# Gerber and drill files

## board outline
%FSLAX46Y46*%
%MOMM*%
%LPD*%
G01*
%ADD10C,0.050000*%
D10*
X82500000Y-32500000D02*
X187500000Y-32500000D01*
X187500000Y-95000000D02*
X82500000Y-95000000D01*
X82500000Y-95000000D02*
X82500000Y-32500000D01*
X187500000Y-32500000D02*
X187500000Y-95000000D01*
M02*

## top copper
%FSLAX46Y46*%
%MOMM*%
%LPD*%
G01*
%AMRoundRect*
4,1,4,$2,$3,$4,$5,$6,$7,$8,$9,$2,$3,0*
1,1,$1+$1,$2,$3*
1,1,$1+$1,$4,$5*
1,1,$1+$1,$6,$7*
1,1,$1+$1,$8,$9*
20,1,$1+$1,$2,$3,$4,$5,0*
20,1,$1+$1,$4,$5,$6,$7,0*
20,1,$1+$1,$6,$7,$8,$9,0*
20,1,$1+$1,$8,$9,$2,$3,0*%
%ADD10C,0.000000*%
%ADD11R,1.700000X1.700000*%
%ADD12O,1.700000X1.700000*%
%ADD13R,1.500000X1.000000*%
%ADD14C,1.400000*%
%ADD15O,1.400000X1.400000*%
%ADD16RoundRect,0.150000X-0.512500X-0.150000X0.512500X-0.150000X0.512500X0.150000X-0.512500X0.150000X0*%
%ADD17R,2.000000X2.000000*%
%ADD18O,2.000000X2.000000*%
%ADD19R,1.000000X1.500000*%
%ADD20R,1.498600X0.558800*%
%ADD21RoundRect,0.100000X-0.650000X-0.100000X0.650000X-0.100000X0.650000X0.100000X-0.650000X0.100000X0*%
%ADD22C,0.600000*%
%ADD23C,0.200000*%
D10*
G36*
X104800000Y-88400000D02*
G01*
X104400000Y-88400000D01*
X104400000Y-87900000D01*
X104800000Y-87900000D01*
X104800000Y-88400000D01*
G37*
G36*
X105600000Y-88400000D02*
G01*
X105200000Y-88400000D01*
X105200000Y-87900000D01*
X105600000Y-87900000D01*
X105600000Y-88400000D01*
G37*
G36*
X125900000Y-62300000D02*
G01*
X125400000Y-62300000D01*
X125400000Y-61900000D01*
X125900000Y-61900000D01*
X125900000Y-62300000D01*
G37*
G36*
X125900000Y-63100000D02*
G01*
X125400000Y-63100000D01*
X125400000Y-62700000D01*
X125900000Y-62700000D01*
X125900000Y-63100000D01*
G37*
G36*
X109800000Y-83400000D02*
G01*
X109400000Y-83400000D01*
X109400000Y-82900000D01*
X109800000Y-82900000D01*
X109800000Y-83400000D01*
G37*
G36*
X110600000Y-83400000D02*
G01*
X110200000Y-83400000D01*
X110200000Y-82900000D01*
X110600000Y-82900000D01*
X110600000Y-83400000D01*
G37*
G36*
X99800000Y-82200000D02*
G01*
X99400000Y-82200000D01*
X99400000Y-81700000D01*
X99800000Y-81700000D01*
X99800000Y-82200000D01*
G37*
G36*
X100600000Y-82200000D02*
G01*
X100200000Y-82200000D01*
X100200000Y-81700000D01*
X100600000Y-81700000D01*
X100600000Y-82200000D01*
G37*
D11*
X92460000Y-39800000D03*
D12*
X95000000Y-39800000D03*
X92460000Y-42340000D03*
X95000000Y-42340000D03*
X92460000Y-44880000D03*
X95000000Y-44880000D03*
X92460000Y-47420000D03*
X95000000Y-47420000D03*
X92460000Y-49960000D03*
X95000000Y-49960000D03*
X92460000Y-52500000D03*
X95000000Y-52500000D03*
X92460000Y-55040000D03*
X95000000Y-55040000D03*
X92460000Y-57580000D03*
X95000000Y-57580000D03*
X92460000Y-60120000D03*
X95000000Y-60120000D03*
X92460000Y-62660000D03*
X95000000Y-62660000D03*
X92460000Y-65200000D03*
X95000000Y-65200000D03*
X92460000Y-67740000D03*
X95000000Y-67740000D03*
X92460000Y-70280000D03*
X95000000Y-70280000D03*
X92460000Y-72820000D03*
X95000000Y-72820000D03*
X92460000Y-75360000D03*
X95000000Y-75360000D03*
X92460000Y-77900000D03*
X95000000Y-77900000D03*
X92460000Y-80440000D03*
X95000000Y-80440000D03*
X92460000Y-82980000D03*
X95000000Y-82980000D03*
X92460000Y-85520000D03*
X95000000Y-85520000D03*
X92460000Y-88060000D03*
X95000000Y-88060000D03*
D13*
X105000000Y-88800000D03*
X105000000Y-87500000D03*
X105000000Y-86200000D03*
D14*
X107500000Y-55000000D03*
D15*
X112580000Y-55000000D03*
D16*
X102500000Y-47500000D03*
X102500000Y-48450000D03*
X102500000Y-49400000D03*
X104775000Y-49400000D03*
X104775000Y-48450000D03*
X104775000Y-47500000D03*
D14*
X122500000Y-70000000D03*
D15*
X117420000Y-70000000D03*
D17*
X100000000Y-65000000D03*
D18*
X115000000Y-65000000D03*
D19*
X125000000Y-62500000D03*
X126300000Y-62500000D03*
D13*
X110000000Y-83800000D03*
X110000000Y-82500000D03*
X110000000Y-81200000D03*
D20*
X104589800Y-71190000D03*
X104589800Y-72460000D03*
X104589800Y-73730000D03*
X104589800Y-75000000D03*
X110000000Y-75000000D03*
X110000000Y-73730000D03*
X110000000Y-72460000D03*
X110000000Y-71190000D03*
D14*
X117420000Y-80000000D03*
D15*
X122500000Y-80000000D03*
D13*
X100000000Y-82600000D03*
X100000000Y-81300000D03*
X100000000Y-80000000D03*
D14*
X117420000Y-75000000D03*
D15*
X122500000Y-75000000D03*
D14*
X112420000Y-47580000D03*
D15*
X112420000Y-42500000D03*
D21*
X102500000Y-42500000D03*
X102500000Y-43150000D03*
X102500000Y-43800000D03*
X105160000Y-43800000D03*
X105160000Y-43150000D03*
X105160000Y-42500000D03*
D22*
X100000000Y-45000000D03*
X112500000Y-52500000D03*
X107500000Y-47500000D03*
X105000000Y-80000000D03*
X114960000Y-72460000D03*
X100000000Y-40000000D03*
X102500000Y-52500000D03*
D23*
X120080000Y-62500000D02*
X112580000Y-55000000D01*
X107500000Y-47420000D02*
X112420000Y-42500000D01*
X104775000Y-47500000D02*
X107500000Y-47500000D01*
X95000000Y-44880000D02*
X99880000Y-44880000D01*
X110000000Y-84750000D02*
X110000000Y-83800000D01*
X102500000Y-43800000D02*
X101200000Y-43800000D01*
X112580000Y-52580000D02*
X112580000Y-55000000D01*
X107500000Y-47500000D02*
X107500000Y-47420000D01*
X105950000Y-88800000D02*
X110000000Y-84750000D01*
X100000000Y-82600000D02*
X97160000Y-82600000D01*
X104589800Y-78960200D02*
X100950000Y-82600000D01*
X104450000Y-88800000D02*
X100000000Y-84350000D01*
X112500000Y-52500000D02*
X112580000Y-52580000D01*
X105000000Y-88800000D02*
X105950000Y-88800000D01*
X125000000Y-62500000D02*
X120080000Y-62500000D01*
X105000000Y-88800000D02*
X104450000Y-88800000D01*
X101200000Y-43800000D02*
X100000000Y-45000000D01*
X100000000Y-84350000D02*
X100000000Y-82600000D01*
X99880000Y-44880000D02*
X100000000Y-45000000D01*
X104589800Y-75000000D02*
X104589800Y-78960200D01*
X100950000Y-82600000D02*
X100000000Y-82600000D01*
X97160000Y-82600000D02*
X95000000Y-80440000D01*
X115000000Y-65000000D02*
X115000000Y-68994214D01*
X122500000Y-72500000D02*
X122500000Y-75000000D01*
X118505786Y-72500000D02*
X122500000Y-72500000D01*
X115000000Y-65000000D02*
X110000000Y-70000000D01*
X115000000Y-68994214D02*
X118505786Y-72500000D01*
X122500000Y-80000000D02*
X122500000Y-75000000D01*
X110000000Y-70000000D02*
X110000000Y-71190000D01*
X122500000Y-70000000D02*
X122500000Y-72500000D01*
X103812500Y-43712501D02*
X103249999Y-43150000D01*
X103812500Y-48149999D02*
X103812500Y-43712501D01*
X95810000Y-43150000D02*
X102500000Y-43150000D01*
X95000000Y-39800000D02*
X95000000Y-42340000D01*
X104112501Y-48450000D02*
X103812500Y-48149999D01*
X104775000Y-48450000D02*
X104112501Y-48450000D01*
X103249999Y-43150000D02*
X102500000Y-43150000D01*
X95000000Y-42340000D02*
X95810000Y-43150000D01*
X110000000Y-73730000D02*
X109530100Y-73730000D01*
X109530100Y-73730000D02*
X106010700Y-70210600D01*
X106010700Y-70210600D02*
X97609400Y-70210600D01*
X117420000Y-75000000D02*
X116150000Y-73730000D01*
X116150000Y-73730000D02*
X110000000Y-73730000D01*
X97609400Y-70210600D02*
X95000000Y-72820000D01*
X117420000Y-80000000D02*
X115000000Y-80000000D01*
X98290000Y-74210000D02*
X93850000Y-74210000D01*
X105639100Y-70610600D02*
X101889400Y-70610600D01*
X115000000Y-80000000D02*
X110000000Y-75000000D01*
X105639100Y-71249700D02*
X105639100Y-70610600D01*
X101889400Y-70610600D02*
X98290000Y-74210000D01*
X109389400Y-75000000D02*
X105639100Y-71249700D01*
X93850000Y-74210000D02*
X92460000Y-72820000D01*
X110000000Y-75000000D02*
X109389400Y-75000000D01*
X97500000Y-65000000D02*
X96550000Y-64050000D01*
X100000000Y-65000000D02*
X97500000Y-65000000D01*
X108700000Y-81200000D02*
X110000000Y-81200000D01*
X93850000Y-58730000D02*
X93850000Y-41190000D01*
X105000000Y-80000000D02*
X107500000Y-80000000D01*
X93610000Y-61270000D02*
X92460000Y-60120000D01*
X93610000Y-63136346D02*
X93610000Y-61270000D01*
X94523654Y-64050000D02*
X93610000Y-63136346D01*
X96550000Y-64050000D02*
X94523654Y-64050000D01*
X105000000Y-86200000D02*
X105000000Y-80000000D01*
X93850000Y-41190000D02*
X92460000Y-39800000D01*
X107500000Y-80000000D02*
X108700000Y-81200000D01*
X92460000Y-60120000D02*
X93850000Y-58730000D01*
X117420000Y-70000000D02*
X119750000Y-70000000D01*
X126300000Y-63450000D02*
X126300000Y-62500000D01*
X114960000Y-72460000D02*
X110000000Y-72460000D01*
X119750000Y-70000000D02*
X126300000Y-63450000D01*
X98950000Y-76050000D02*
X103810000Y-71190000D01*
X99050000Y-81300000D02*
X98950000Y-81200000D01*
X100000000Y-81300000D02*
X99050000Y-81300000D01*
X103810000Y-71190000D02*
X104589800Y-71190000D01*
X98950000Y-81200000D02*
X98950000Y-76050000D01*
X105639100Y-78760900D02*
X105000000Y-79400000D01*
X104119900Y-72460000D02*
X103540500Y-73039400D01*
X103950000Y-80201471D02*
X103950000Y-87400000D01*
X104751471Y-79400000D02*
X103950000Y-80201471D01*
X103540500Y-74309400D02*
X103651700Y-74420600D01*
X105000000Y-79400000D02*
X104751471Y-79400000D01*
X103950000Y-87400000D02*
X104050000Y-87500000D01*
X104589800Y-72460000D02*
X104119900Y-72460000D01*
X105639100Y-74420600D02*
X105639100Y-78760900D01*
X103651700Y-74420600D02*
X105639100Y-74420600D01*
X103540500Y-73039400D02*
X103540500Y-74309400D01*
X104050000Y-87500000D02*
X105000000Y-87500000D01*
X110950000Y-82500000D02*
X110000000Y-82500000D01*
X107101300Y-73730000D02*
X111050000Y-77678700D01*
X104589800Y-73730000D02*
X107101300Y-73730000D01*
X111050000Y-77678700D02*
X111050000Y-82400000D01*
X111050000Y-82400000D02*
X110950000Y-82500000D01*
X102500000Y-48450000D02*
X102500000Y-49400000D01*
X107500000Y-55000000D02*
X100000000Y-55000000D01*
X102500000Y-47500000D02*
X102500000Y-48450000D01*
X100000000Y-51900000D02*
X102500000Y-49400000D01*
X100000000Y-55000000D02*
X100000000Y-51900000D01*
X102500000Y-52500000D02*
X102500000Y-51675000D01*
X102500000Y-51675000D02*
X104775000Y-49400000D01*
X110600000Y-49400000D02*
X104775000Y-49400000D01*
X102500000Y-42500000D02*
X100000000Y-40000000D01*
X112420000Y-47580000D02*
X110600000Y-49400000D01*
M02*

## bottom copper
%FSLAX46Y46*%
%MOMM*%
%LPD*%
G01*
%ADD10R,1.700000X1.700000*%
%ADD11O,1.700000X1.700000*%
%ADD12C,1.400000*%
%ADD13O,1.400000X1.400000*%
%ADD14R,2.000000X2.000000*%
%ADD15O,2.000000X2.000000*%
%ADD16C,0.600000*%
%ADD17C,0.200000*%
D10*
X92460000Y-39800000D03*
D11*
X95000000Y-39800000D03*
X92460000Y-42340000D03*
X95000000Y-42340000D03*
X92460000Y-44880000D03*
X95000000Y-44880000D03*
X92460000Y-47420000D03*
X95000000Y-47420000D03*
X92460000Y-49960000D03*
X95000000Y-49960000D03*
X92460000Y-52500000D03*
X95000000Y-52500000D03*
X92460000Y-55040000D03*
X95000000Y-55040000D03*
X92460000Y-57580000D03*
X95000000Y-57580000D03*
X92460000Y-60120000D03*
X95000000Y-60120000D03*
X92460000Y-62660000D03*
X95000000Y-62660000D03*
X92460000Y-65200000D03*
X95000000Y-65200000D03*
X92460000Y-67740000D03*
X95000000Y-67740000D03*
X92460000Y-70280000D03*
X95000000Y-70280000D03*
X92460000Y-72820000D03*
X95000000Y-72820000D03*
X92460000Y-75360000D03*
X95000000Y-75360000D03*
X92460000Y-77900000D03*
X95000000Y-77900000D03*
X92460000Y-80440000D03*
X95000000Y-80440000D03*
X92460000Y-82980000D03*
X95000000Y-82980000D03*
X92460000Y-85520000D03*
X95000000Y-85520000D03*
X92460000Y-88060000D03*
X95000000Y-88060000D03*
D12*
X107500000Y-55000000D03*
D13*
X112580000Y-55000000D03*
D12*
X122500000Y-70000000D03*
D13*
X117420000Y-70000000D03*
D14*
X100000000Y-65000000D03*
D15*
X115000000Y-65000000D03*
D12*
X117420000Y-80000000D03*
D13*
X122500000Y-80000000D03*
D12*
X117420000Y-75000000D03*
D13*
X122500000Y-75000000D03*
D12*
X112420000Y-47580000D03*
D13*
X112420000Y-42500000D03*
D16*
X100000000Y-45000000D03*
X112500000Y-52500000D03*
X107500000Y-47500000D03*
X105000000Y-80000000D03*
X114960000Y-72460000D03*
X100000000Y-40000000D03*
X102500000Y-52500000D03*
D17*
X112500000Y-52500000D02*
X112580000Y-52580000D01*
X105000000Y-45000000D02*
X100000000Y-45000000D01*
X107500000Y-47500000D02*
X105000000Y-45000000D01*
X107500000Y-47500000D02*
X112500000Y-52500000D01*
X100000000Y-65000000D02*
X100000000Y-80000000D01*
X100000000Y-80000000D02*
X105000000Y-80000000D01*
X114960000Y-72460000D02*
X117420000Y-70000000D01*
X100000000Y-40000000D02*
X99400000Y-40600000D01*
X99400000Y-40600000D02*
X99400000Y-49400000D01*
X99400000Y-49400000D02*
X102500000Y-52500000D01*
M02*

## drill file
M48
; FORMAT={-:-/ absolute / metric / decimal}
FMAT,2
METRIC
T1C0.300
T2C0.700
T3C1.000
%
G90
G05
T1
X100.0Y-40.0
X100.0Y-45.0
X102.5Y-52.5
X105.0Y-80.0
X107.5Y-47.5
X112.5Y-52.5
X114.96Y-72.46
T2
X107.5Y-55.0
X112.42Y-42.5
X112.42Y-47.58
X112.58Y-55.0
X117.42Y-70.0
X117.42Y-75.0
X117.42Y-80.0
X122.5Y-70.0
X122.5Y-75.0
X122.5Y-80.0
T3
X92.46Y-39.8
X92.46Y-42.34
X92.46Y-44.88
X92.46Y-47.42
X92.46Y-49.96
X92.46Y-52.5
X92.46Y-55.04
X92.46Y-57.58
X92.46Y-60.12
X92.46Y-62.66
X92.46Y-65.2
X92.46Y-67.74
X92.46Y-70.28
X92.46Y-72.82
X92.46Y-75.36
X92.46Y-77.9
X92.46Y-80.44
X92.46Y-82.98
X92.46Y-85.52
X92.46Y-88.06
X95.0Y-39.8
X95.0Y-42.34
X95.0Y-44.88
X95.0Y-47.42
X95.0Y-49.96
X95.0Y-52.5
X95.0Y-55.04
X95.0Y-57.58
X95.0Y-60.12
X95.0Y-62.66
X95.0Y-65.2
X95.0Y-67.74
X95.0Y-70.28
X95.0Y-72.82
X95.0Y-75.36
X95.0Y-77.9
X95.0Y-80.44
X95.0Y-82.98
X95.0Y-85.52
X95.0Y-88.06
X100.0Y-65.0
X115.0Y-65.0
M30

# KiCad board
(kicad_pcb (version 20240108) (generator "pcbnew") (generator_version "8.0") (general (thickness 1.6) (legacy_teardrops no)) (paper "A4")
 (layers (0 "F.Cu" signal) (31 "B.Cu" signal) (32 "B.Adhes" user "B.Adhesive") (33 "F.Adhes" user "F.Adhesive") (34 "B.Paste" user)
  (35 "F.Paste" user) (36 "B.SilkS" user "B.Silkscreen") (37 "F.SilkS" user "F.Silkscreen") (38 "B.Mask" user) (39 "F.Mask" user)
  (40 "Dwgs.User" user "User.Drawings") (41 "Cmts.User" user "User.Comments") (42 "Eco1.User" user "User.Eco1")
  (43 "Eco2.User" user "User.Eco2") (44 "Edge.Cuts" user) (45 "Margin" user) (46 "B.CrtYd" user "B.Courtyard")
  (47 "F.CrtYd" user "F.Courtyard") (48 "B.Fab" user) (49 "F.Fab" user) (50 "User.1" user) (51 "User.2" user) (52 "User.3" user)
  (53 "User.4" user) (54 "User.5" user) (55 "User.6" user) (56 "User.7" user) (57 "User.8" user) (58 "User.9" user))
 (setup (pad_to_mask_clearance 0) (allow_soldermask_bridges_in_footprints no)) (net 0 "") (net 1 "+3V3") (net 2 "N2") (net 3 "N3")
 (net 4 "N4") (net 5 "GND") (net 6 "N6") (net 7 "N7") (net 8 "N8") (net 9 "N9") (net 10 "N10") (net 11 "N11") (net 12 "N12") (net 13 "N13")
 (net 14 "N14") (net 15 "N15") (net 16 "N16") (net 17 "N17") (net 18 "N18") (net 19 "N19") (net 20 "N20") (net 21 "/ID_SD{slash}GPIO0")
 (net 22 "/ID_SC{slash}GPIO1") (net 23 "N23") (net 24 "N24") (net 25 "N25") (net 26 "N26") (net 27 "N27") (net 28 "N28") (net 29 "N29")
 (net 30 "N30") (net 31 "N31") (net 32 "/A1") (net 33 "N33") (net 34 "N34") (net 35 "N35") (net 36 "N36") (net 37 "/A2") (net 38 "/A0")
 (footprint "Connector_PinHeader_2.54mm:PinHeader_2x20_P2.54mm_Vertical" (layer "F.Cu") (at 92.46 39.8)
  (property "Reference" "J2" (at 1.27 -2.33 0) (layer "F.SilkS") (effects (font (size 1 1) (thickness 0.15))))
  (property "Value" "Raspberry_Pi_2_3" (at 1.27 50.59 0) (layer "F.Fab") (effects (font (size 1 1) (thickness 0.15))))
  (pad "1" thru_hole rect (at 0 0) (size 1.7 1.7) (drill 1) (layers "*.Cu" "*.Mask") (remove_unused_layers no) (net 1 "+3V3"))
  (pad "2" thru_hole oval (at 2.54 0) (size 1.7 1.7) (drill 1) (layers "*.Cu" "*.Mask") (remove_unused_layers no) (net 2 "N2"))
  (pad "3" thru_hole oval (at 0 2.54) (size 1.7 1.7) (drill 1) (layers "*.Cu" "*.Mask") (remove_unused_layers no) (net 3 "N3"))
  (pad "4" thru_hole oval (at 2.54 2.54) (size 1.7 1.7) (drill 1) (layers "*.Cu" "*.Mask") (remove_unused_layers no) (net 2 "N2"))
  (pad "5" thru_hole oval (at 0 5.08) (size 1.7 1.7) (drill 1) (layers "*.Cu" "*.Mask") (remove_unused_layers no) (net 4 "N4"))
  (pad "6" thru_hole oval (at 2.54 5.08) (size 1.7 1.7) (drill 1) (layers "*.Cu" "*.Mask") (remove_unused_layers no) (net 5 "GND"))
  (pad "7" thru_hole oval (at 0 7.62) (size 1.7 1.7) (drill 1) (layers "*.Cu" "*.Mask") (remove_unused_layers no) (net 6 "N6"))
  (pad "8" thru_hole oval (at 2.54 7.62) (size 1.7 1.7) (drill 1) (layers "*.Cu" "*.Mask") (remove_unused_layers no) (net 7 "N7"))
  (pad "9" thru_hole oval (at 0 10.16) (size 1.7 1.7) (drill 1) (layers "*.Cu" "*.Mask") (remove_unused_layers no) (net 5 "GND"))
  (pad "10" thru_hole oval (at 2.54 10.16) (size 1.7 1.7) (drill 1) (layers "*.Cu" "*.Mask") (remove_unused_layers no) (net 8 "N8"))
  (pad "11" thru_hole oval (at 0 12.7) (size 1.7 1.7) (drill 1) (layers "*.Cu" "*.Mask") (remove_unused_layers no) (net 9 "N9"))
  (pad "12" thru_hole oval (at 2.54 12.7) (size 1.7 1.7) (drill 1) (layers "*.Cu" "*.Mask") (remove_unused_layers no) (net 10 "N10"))
  (pad "13" thru_hole oval (at 0 15.24) (size 1.7 1.7) (drill 1) (layers "*.Cu" "*.Mask") (remove_unused_layers no) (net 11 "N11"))
  (pad "14" thru_hole oval (at 2.54 15.24) (size 1.7 1.7) (drill 1) (layers "*.Cu" "*.Mask") (remove_unused_layers no) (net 5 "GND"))
  (pad "15" thru_hole oval (at 0 17.78) (size 1.7 1.7) (drill 1) (layers "*.Cu" "*.Mask") (remove_unused_layers no) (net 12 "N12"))
  (pad "16" thru_hole oval (at 2.54 17.78) (size 1.7 1.7) (drill 1) (layers "*.Cu" "*.Mask") (remove_unused_layers no) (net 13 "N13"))
  (pad "17" thru_hole oval (at 0 20.32) (size 1.7 1.7) (drill 1) (layers "*.Cu" "*.Mask") (remove_unused_layers no) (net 1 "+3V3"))
  (pad "18" thru_hole oval (at 2.54 20.32) (size 1.7 1.7) (drill 1) (layers "*.Cu" "*.Mask") (remove_unused_layers no) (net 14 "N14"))
  (pad "19" thru_hole oval (at 0 22.86) (size 1.7 1.7) (drill 1) (layers "*.Cu" "*.Mask") (remove_unused_layers no) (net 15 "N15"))
  (pad "20" thru_hole oval (at 2.54 22.86) (size 1.7 1.7) (drill 1) (layers "*.Cu" "*.Mask") (remove_unused_layers no) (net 5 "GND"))
  (pad "21" thru_hole oval (at 0 25.4) (size 1.7 1.7) (drill 1) (layers "*.Cu" "*.Mask") (remove_unused_layers no) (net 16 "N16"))
  (pad "22" thru_hole oval (at 2.54 25.4) (size 1.7 1.7) (drill 1) (layers "*.Cu" "*.Mask") (remove_unused_layers no) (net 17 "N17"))
  (pad "23" thru_hole oval (at 0 27.94) (size 1.7 1.7) (drill 1) (layers "*.Cu" "*.Mask") (remove_unused_layers no) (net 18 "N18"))
  (pad "24" thru_hole oval (at 2.54 27.94) (size 1.7 1.7) (drill 1) (layers "*.Cu" "*.Mask") (remove_unused_layers no) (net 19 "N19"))
  (pad "25" thru_hole oval (at 0 30.48) (size 1.7 1.7) (drill 1) (layers "*.Cu" "*.Mask") (remove_unused_layers no) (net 5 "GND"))
  (pad "26" thru_hole oval (at 2.54 30.48) (size 1.7 1.7) (drill 1) (layers "*.Cu" "*.Mask") (remove_unused_layers no) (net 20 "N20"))
  (pad "27" thru_hole oval (at 0 33.02) (size 1.7 1.7) (drill 1) (layers "*.Cu" "*.Mask") (remove_unused_layers no)
   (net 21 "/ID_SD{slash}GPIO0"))
  (pad "28" thru_hole oval (at 2.54 33.02) (size 1.7 1.7) (drill 1) (layers "*.Cu" "*.Mask") (remove_unused_layers no)
   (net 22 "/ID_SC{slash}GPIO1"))
  (pad "29" thru_hole oval (at 0 35.56) (size 1.7 1.7) (drill 1) (layers "*.Cu" "*.Mask") (remove_unused_layers no) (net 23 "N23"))
  (pad "30" thru_hole oval (at 2.54 35.56) (size 1.7 1.7) (drill 1) (layers "*.Cu" "*.Mask") (remove_unused_layers no) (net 5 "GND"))
  (pad "31" thru_hole oval (at 0 38.1) (size 1.7 1.7) (drill 1) (layers "*.Cu" "*.Mask") (remove_unused_layers no) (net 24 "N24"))
  (pad "32" thru_hole oval (at 2.54 38.1) (size 1.7 1.7) (drill 1) (layers "*.Cu" "*.Mask") (remove_unused_layers no) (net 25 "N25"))
  (pad "33" thru_hole oval (at 0 40.64) (size 1.7 1.7) (drill 1) (layers "*.Cu" "*.Mask") (remove_unused_layers no) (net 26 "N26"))
  (pad "34" thru_hole oval (at 2.54 40.64) (size 1.7 1.7) (drill 1) (layers "*.Cu" "*.Mask") (remove_unused_layers no) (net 5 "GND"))
  (pad "35" thru_hole oval (at 0 43.18) (size 1.7 1.7) (drill 1) (layers "*.Cu" "*.Mask") (remove_unused_layers no) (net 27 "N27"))
  (pad "36" thru_hole oval (at 2.54 43.18) (size 1.7 1.7) (drill 1) (layers "*.Cu" "*.Mask") (remove_unused_layers no) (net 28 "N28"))
  (pad "37" thru_hole oval (at 0 45.72) (size 1.7 1.7) (drill 1) (layers "*.Cu" "*.Mask") (remove_unused_layers no) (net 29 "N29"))
  (pad "38" thru_hole oval (at 2.54 45.72) (size 1.7 1.7) (drill 1) (layers "*.Cu" "*.Mask") (remove_unused_layers no) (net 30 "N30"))
  (pad "39" thru_hole oval (at 0 48.26) (size 1.7 1.7) (drill 1) (layers "*.Cu" "*.Mask") (remove_unused_layers no) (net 5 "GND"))
  (pad "40" thru_hole oval (at 2.54 48.26) (size 1.7 1.7) (drill 1) (layers "*.Cu" "*.Mask") (remove_unused_layers no) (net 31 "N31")))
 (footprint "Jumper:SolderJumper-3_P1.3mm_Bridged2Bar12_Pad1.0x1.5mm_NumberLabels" (layer "F.Cu") (at 105 87.5 90)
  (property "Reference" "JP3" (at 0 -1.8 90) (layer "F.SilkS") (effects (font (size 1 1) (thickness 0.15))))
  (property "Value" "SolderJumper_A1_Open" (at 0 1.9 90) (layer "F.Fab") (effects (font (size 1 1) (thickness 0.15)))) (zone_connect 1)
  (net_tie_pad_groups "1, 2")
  (fp_poly (pts (xy -0.9 -0.6) (xy -0.4 -0.6) (xy -0.4 -0.2) (xy -0.9 -0.2)) (stroke (width 0) (type solid)) (fill solid) (layer "F.Cu"))
  (fp_poly (pts (xy -0.9 0.2) (xy -0.4 0.2) (xy -0.4 0.6) (xy -0.9 0.6)) (stroke (width 0) (type solid)) (fill solid) (layer "F.Cu"))
  (pad "1" smd rect (at -1.3 0 90) (size 1 1.5) (layers "F.Cu" "F.Mask") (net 5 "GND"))
  (pad "2" smd rect (at 0 0 90) (size 1 1.5) (layers "F.Cu" "F.Mask") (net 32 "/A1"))
  (pad "3" smd rect (at 1.3 0 90) (size 1 1.5) (layers "F.Cu" "F.Mask") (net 1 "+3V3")))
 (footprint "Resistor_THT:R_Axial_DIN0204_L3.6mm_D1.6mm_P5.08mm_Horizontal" (layer "F.Cu") (at 107.5 55)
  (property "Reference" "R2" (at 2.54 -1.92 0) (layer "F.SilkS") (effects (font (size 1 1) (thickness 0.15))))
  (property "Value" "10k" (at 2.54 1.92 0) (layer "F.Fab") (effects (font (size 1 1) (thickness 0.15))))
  (pad "1" thru_hole circle (at 0 0) (size 1.4 1.4) (drill 0.7) (layers "*.Cu" "*.Mask") (remove_unused_layers no) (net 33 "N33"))
  (pad "2" thru_hole oval (at 5.08 0) (size 1.4 1.4) (drill 0.7) (layers "*.Cu" "*.Mask") (remove_unused_layers no) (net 5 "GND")))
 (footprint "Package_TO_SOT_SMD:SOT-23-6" (layer "F.Cu") (at 103.6375 48.45)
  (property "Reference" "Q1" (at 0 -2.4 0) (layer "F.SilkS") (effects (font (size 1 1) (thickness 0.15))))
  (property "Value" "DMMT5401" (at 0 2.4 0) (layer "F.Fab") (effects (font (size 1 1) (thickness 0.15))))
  (pad "1" smd roundrect (at -1.1375 -0.95) (size 1.325 0.6) (layers "F.Cu" "F.Paste" "F.Mask") (roundrect_rratio 0.25) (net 33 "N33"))
  (pad "2" smd roundrect (at -1.1375 0) (size 1.325 0.6) (layers "F.Cu" "F.Paste" "F.Mask") (roundrect_rratio 0.25) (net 33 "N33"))
  (pad "3" smd roundrect (at -1.1375 0.95) (size 1.325 0.6) (layers "F.Cu" "F.Paste" "F.Mask") (roundrect_rratio 0.25) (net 33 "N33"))
  (pad "4" smd roundrect (at 1.1375 0.95) (size 1.325 0.6) (layers "F.Cu" "F.Paste" "F.Mask") (roundrect_rratio 0.25) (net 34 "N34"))
  (pad "5" smd roundrect (at 1.1375 0) (size 1.325 0.6) (layers "F.Cu" "F.Paste" "F.Mask") (roundrect_rratio 0.25) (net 2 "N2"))
  (pad "6" smd roundrect (at 1.1375 -0.95) (size 1.325 0.6) (layers "F.Cu" "F.Paste" "F.Mask") (roundrect_rratio 0.25) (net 5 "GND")))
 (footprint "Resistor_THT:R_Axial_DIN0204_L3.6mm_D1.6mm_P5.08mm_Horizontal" (layer "F.Cu") (at 122.5 70 180)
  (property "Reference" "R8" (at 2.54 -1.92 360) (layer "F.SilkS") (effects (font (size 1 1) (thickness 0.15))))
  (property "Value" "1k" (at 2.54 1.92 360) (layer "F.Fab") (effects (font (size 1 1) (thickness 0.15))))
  (pad "1" thru_hole circle (at 0 0 180) (size 1.4 1.4) (drill 0.7) (layers "*.Cu" "*.Mask") (remove_unused_layers no) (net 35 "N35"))
  (pad "2" thru_hole oval (at 5.08 0 180) (size 1.4 1.4) (drill 0.7) (layers "*.Cu" "*.Mask") (remove_unused_layers no) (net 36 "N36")))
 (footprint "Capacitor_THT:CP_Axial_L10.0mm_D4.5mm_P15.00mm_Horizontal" (layer "F.Cu") (at 100 65)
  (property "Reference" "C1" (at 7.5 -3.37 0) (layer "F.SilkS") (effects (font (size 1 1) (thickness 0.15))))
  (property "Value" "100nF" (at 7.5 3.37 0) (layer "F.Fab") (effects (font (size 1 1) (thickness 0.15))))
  (pad "1" thru_hole rect (at 0 0) (size 2 2) (drill 1) (layers "*.Cu" "*.Mask") (remove_unused_layers no) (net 1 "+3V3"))
  (pad "2" thru_hole oval (at 15 0) (size 2 2) (drill 1) (layers "*.Cu" "*.Mask") (remove_unused_layers no) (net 35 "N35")))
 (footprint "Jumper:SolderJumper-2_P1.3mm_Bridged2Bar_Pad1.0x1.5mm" (layer "F.Cu") (at 125.65 62.5)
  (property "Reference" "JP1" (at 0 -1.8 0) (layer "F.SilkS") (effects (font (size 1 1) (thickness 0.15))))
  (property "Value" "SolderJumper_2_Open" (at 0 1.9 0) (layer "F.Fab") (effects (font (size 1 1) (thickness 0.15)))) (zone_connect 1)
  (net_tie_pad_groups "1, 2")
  (fp_poly (pts (xy -0.25 -0.6) (xy 0.25 -0.6) (xy 0.25 -0.2) (xy -0.25 -0.2)) (stroke (width 0) (type solid)) (fill solid) (layer "F.Cu"))
  (fp_poly (pts (xy -0.25 0.2) (xy 0.25 0.2) (xy 0.25 0.6) (xy -0.25 0.6)) (stroke (width 0) (type solid)) (fill solid) (layer "F.Cu"))
  (pad "1" smd rect (at -0.65 0) (size 1 1.5) (layers "F.Cu" "F.Mask") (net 5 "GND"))
  (pad "2" smd rect (at 0.65 0) (size 1 1.5) (layers "F.Cu" "F.Mask") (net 36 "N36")))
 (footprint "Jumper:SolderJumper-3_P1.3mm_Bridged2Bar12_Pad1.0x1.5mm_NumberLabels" (layer "F.Cu") (at 110 82.5 90)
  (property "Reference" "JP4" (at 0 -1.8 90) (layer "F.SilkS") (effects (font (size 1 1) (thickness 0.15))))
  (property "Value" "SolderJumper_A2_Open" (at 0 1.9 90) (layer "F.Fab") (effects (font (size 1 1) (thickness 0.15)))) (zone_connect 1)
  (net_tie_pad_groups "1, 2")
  (fp_poly (pts (xy -0.9 -0.6) (xy -0.4 -0.6) (xy -0.4 -0.2) (xy -0.9 -0.2)) (stroke (width 0) (type solid)) (fill solid) (layer "F.Cu"))
  (fp_poly (pts (xy -0.9 0.2) (xy -0.4 0.2) (xy -0.4 0.6) (xy -0.9 0.6)) (stroke (width 0) (type solid)) (fill solid) (layer "F.Cu"))
  (pad "1" smd rect (at -1.3 0 90) (size 1 1.5) (layers "F.Cu" "F.Mask") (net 5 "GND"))
  (pad "2" smd rect (at 0 0 90) (size 1 1.5) (layers "F.Cu" "F.Mask") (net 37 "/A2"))
  (pad "3" smd rect (at 1.3 0 90) (size 1 1.5) (layers "F.Cu" "F.Mask") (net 1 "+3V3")))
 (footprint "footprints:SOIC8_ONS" (layer "F.Cu") (at 107.2949 73.095)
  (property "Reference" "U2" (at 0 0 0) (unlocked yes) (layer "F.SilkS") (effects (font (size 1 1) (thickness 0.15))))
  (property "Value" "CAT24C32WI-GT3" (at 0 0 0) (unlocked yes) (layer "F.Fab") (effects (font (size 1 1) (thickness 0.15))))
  (pad "1" smd rect (at -2.7051 -1.905) (size 1.4986 0.5588) (layers "F.Cu" "F.Paste" "F.Mask") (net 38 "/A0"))
  (pad "2" smd rect (at -2.7051 -0.635) (size 1.4986 0.5588) (layers "F.Cu" "F.Paste" "F.Mask") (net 32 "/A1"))
  (pad "3" smd rect (at -2.7051 0.635) (size 1.4986 0.5588) (layers "F.Cu" "F.Paste" "F.Mask") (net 37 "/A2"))
  (pad "4" smd rect (at -2.7051 1.905) (size 1.4986 0.5588) (layers "F.Cu" "F.Paste" "F.Mask") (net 5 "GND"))
  (pad "5" smd rect (at 2.7051 1.905) (size 1.4986 0.5588) (layers "F.Cu" "F.Paste" "F.Mask") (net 21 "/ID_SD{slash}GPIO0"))
  (pad "6" smd rect (at 2.7051 0.635) (size 1.4986 0.5588) (layers "F.Cu" "F.Paste" "F.Mask") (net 22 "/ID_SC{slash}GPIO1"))
  (pad "7" smd rect (at 2.7051 -0.635) (size 1.4986 0.5588) (layers "F.Cu" "F.Paste" "F.Mask") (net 36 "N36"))
  (pad "8" smd rect (at 2.7051 -1.905) (size 1.4986 0.5588) (layers "F.Cu" "F.Paste" "F.Mask") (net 35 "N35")))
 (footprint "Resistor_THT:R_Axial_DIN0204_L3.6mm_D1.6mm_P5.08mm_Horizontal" (layer "F.Cu") (at 117.42 80)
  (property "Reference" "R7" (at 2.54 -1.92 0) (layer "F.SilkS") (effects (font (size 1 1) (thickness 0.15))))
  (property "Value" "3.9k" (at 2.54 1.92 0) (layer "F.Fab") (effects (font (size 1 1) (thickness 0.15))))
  (pad "1" thru_hole circle (at 0 0) (size 1.4 1.4) (drill 0.7) (layers "*.Cu" "*.Mask") (remove_unused_layers no)
   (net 21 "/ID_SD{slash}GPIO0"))
  (pad "2" thru_hole oval (at 5.08 0) (size 1.4 1.4) (drill 0.7) (layers "*.Cu" "*.Mask") (remove_unused_layers no) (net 35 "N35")))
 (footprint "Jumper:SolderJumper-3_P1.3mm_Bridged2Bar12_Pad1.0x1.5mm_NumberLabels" (layer "F.Cu") (at 100 81.3 90)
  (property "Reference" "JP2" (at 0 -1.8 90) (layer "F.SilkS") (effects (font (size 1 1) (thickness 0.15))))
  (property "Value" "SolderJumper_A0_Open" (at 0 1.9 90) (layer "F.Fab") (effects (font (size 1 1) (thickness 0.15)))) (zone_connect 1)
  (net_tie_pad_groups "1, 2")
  (fp_poly (pts (xy -0.9 -0.6) (xy -0.4 -0.6) (xy -0.4 -0.2) (xy -0.9 -0.2)) (stroke (width 0) (type solid)) (fill solid) (layer "F.Cu"))
  (fp_poly (pts (xy -0.9 0.2) (xy -0.4 0.2) (xy -0.4 0.6) (xy -0.9 0.6)) (stroke (width 0) (type solid)) (fill solid) (layer "F.Cu"))
  (pad "1" smd rect (at -1.3 0 90) (size 1 1.5) (layers "F.Cu" "F.Mask") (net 5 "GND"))
  (pad "2" smd rect (at 0 0 90) (size 1 1.5) (layers "F.Cu" "F.Mask") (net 38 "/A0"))
  (pad "3" smd rect (at 1.3 0 90) (size 1 1.5) (layers "F.Cu" "F.Mask") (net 1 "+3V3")))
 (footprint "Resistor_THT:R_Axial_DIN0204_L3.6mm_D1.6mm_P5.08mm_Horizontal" (layer "F.Cu") (at 117.42 75)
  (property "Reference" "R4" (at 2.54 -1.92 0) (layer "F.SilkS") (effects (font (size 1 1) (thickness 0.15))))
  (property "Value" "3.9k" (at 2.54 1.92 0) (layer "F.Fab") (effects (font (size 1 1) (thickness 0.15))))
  (pad "1" thru_hole circle (at 0 0) (size 1.4 1.4) (drill 0.7) (layers "*.Cu" "*.Mask") (remove_unused_layers no)
   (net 22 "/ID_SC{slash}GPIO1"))
  (pad "2" thru_hole oval (at 5.08 0) (size 1.4 1.4) (drill 0.7) (layers "*.Cu" "*.Mask") (remove_unused_layers no) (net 35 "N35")))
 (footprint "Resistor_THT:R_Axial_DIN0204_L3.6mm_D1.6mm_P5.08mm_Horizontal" (layer "F.Cu") (at 112.42 47.58 90)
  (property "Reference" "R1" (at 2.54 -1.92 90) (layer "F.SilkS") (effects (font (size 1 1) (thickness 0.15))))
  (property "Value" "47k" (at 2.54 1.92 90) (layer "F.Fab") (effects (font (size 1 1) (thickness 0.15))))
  (pad "1" thru_hole circle (at 0 0 90) (size 1.4 1.4) (drill 0.7) (layers "*.Cu" "*.Mask") (remove_unused_layers no) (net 34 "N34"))
  (pad "2" thru_hole oval (at 5.08 0 90) (size 1.4 1.4) (drill 0.7) (layers "*.Cu" "*.Mask") (remove_unused_layers no) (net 5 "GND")))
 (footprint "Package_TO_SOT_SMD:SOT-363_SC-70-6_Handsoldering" (layer "F.Cu") (at 103.83 43.15)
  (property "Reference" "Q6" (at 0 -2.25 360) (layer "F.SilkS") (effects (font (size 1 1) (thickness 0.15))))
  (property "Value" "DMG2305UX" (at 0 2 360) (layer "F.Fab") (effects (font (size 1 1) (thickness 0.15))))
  (pad "1" smd roundrect (at -1.33 -0.65) (size 1.5 0.4) (layers "F.Cu" "F.Paste" "F.Mask") (roundrect_rratio 0.25) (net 34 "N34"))
  (pad "2" smd roundrect (at -1.33 0) (size 1.5 0.4) (layers "F.Cu" "F.Paste" "F.Mask") (roundrect_rratio 0.25) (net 2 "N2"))
  (pad "3" smd roundrect (at -1.33 0.65) (size 1.5 0.4) (layers "F.Cu" "F.Paste" "F.Mask") (roundrect_rratio 0.25) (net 5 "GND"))
  (pad "4" smd roundrect (at 1.33 0.65) (size 1.5 0.4) (layers "F.Cu" "F.Paste" "F.Mask") (roundrect_rratio 0.25))
  (pad "5" smd roundrect (at 1.33 0) (size 1.5 0.4) (layers "F.Cu" "F.Paste" "F.Mask") (roundrect_rratio 0.25))
  (pad "6" smd roundrect (at 1.33 -0.65) (size 1.5 0.4) (layers "F.Cu" "F.Paste" "F.Mask") (roundrect_rratio 0.25)))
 (gr_line (start 82.5 32.5) (end 187.5 32.5) (stroke (width 0.05) (type default)) (layer "Edge.Cuts"))
 (gr_line (start 187.5 95) (end 82.5 95) (stroke (width 0.05) (type default)) (layer "Edge.Cuts"))
 (gr_line (start 82.5 95) (end 82.5 32.5) (stroke (width 0.05) (type default)) (layer "Edge.Cuts"))
 (gr_line (start 187.5 32.5) (end 187.5 95) (stroke (width 0.05) (type default)) (layer "Edge.Cuts"))
 (segment (start 120.08 62.5) (end 112.58 55) (width 0.2) (layer "F.Cu") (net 5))
 (segment (start 107.5 47.42) (end 112.42 42.5) (width 0.2) (layer "F.Cu") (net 5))
 (segment (start 104.775 47.5) (end 107.5 47.5) (width 0.2) (layer "F.Cu") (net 5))
 (segment (start 95 44.88) (end 99.88 44.88) (width 0.2) (layer "F.Cu") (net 5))
 (segment (start 110 84.75) (end 110 83.8) (width 0.2) (layer "F.Cu") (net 5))
 (segment (start 102.5 43.8) (end 101.2 43.8) (width 0.2) (layer "F.Cu") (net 5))
 (segment (start 112.58 52.58) (end 112.58 55) (width 0.2) (layer "F.Cu") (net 5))
 (segment (start 107.5 47.5) (end 107.5 47.42) (width 0.2) (layer "F.Cu") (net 5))
 (segment (start 105.95 88.8) (end 110 84.75) (width 0.2) (layer "F.Cu") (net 5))
 (segment (start 100 82.6) (end 97.16 82.6) (width 0.2) (layer "F.Cu") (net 5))
 (segment (start 104.5898 78.9602) (end 100.95 82.6) (width 0.2) (layer "F.Cu") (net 5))
 (segment (start 104.45 88.8) (end 100 84.35) (width 0.2) (layer "F.Cu") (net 5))
 (segment (start 112.5 52.5) (end 112.58 52.58) (width 0.2) (layer "F.Cu") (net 5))
 (segment (start 105 88.8) (end 105.95 88.8) (width 0.2) (layer "F.Cu") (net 5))
 (segment (start 125 62.5) (end 120.08 62.5) (width 0.2) (layer "F.Cu") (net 5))
 (segment (start 105 88.8) (end 104.45 88.8) (width 0.2) (layer "F.Cu") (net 5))
 (segment (start 101.2 43.8) (end 100 45) (width 0.2) (layer "F.Cu") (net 5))
 (segment (start 100 84.35) (end 100 82.6) (width 0.2) (layer "F.Cu") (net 5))
 (segment (start 99.88 44.88) (end 100 45) (width 0.2) (layer "F.Cu") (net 5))
 (segment (start 104.5898 75) (end 104.5898 78.9602) (width 0.2) (layer "F.Cu") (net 5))
 (segment (start 100.95 82.6) (end 100 82.6) (width 0.2) (layer "F.Cu") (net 5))
 (segment (start 97.16 82.6) (end 95 80.44) (width 0.2) (layer "F.Cu") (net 5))
 (via (at 100 45) (size 0.6) (drill 0.3) (layers "F.Cu" "B.Cu") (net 5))
 (via (at 112.5 52.5) (size 0.6) (drill 0.3) (layers "F.Cu" "B.Cu") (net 5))
 (via (at 107.5 47.5) (size 0.6) (drill 0.3) (layers "F.Cu" "B.Cu") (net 5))
 (segment (start 112.5 52.5) (end 112.58 52.58) (width 0.2) (layer "B.Cu") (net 5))
 (segment (start 105 45) (end 100 45) (width 0.2) (layer "B.Cu") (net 5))
 (segment (start 107.5 47.5) (end 105 45) (width 0.2) (layer "B.Cu") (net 5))
 (segment (start 107.5 47.5) (end 112.5 52.5) (width 0.2) (layer "B.Cu") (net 5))
 (segment (start 115 65) (end 115 68.994214) (width 0.2) (layer "F.Cu") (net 35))
 (segment (start 122.5 72.5) (end 122.5 75) (width 0.2) (layer "F.Cu") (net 35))
 (segment (start 118.505786 72.5) (end 122.5 72.5) (width 0.2) (layer "F.Cu") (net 35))
 (segment (start 115 65) (end 110 70) (width 0.2) (layer "F.Cu") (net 35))
 (segment (start 115 68.994214) (end 118.505786 72.5) (width 0.2) (layer "F.Cu") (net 35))
 (segment (start 122.5 80) (end 122.5 75) (width 0.2) (layer "F.Cu") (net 35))
 (segment (start 110 70) (end 110 71.19) (width 0.2) (layer "F.Cu") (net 35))
 (segment (start 122.5 70) (end 122.5 72.5) (width 0.2) (layer "F.Cu") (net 35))
 (segment (start 103.8125 43.712501) (end 103.249999 43.15) (width 0.2) (layer "F.Cu") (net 2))
 (segment (start 103.8125 48.149999) (end 103.8125 43.712501) (width 0.2) (layer "F.Cu") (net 2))
 (segment (start 95.81 43.15) (end 102.5 43.15) (width 0.2) (layer "F.Cu") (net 2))
 (segment (start 95 39.8) (end 95 42.34) (width 0.2) (layer "F.Cu") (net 2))
 (segment (start 104.112501 48.45) (end 103.8125 48.149999) (width 0.2) (layer "F.Cu") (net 2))
 (segment (start 104.775 48.45) (end 104.112501 48.45) (width 0.2) (layer "F.Cu") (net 2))
 (segment (start 103.249999 43.15) (end 102.5 43.15) (width 0.2) (layer "F.Cu") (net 2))
 (segment (start 95 42.34) (end 95.81 43.15) (width 0.2) (layer "F.Cu") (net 2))
 (segment (start 110 73.73) (end 109.5301 73.73) (width 0.2) (layer "F.Cu") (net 22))
 (segment (start 109.5301 73.73) (end 106.0107 70.2106) (width 0.2) (layer "F.Cu") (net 22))
 (segment (start 106.0107 70.2106) (end 97.6094 70.2106) (width 0.2) (layer "F.Cu") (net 22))
 (segment (start 117.42 75) (end 116.15 73.73) (width 0.2) (layer "F.Cu") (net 22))
 (segment (start 116.15 73.73) (end 110 73.73) (width 0.2) (layer "F.Cu") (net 22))
 (segment (start 97.6094 70.2106) (end 95 72.82) (width 0.2) (layer "F.Cu") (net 22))
 (segment (start 117.42 80) (end 115 80) (width 0.2) (layer "F.Cu") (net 21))
 (segment (start 98.29 74.21) (end 93.85 74.21) (width 0.2) (layer "F.Cu") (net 21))
 (segment (start 105.6391 70.6106) (end 101.8894 70.6106) (width 0.2) (layer "F.Cu") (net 21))
 (segment (start 115 80) (end 110 75) (width 0.2) (layer "F.Cu") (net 21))
 (segment (start 105.6391 71.2497) (end 105.6391 70.6106) (width 0.2) (layer "F.Cu") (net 21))
 (segment (start 101.8894 70.6106) (end 98.29 74.21) (width 0.2) (layer "F.Cu") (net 21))
 (segment (start 109.3894 75) (end 105.6391 71.2497) (width 0.2) (layer "F.Cu") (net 21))
 (segment (start 93.85 74.21) (end 92.46 72.82) (width 0.2) (layer "F.Cu") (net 21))
 (segment (start 110 75) (end 109.3894 75) (width 0.2) (layer "F.Cu") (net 21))
 (segment (start 97.5 65) (end 96.55 64.05) (width 0.2) (layer "F.Cu") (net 1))
 (segment (start 100 65) (end 97.5 65) (width 0.2) (layer "F.Cu") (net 1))
 (segment (start 108.7 81.2) (end 110 81.2) (width 0.2) (layer "F.Cu") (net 1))
 (segment (start 93.85 58.73) (end 93.85 41.19) (width 0.2) (layer "F.Cu") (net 1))
 (segment (start 105 80) (end 107.5 80) (width 0.2) (layer "F.Cu") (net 1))
 (segment (start 93.61 61.27) (end 92.46 60.12) (width 0.2) (layer "F.Cu") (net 1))
 (segment (start 93.61 63.136346) (end 93.61 61.27) (width 0.2) (layer "F.Cu") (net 1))
 (segment (start 94.523654 64.05) (end 93.61 63.136346) (width 0.2) (layer "F.Cu") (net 1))
 (segment (start 96.55 64.05) (end 94.523654 64.05) (width 0.2) (layer "F.Cu") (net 1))
 (segment (start 105 86.2) (end 105 80) (width 0.2) (layer "F.Cu") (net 1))
 (segment (start 93.85 41.19) (end 92.46 39.8) (width 0.2) (layer "F.Cu") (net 1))
 (segment (start 107.5 80) (end 108.7 81.2) (width 0.2) (layer "F.Cu") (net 1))
 (segment (start 92.46 60.12) (end 93.85 58.73) (width 0.2) (layer "F.Cu") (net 1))
 (via (at 105 80) (size 0.6) (drill 0.3) (layers "F.Cu" "B.Cu") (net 1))
 (segment (start 100 65) (end 100 80) (width 0.2) (layer "B.Cu") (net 1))
 (segment (start 100 80) (end 105 80) (width 0.2) (layer "B.Cu") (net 1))
 (segment (start 117.42 70) (end 119.75 70) (width 0.2) (layer "F.Cu") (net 36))
 (segment (start 126.3 63.45) (end 126.3 62.5) (width 0.2) (layer "F.Cu") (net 36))
 (segment (start 114.96 72.46) (end 110 72.46) (width 0.2) (layer "F.Cu") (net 36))
 (segment (start 119.75 70) (end 126.3 63.45) (width 0.2) (layer "F.Cu") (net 36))
 (via (at 114.96 72.46) (size 0.6) (drill 0.3) (layers "F.Cu" "B.Cu") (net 36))
 (segment (start 114.96 72.46) (end 117.42 70) (width 0.2) (layer "B.Cu") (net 36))
 (segment (start 98.95 76.05) (end 103.81 71.19) (width 0.2) (layer "F.Cu") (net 38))
 (segment (start 99.05 81.3) (end 98.95 81.2) (width 0.2) (layer "F.Cu") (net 38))
 (segment (start 100 81.3) (end 99.05 81.3) (width 0.2) (layer "F.Cu") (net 38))
 (segment (start 103.81 71.19) (end 104.5898 71.19) (width 0.2) (layer "F.Cu") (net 38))
 (segment (start 98.95 81.2) (end 98.95 76.05) (width 0.2) (layer "F.Cu") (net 38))
 (segment (start 105.6391 78.7609) (end 105 79.4) (width 0.2) (layer "F.Cu") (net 32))
 (segment (start 104.1199 72.46) (end 103.5405 73.0394) (width 0.2) (layer "F.Cu") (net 32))
 (segment (start 103.95 80.201471) (end 103.95 87.4) (width 0.2) (layer "F.Cu") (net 32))
 (segment (start 104.751471 79.4) (end 103.95 80.201471) (width 0.2) (layer "F.Cu") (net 32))
 (segment (start 103.5405 74.3094) (end 103.6517 74.4206) (width 0.2) (layer "F.Cu") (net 32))
 (segment (start 105 79.4) (end 104.751471 79.4) (width 0.2) (layer "F.Cu") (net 32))
 (segment (start 103.95 87.4) (end 104.05 87.5) (width 0.2) (layer "F.Cu") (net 32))
 (segment (start 104.5898 72.46) (end 104.1199 72.46) (width 0.2) (layer "F.Cu") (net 32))
 (segment (start 105.6391 74.4206) (end 105.6391 78.7609) (width 0.2) (layer "F.Cu") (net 32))
 (segment (start 103.6517 74.4206) (end 105.6391 74.4206) (width 0.2) (layer "F.Cu") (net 32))
 (segment (start 103.5405 73.0394) (end 103.5405 74.3094) (width 0.2) (layer "F.Cu") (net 32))
 (segment (start 104.05 87.5) (end 105 87.5) (width 0.2) (layer "F.Cu") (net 32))
 (segment (start 110.95 82.5) (end 110 82.5) (width 0.2) (layer "F.Cu") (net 37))
 (segment (start 107.1013 73.73) (end 111.05 77.6787) (width 0.2) (layer "F.Cu") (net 37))
 (segment (start 104.5898 73.73) (end 107.1013 73.73) (width 0.2) (layer "F.Cu") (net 37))
 (segment (start 111.05 77.6787) (end 111.05 82.4) (width 0.2) (layer "F.Cu") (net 37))
 (segment (start 111.05 82.4) (end 110.95 82.5) (width 0.2) (layer "F.Cu") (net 37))
 (segment (start 102.5 48.45) (end 102.5 49.4) (width 0.2) (layer "F.Cu") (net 33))
 (segment (start 107.5 55) (end 100 55) (width 0.2) (layer "F.Cu") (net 33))
 (segment (start 102.5 47.5) (end 102.5 48.45) (width 0.2) (layer "F.Cu") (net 33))
 (segment (start 100 51.9) (end 102.5 49.4) (width 0.2) (layer "F.Cu") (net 33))
 (segment (start 100 55) (end 100 51.9) (width 0.2) (layer "F.Cu") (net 33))
 (segment (start 102.5 52.5) (end 102.5 51.675) (width 0.2) (layer "F.Cu") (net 34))
 (segment (start 102.5 51.675) (end 104.775 49.4) (width 0.2) (layer "F.Cu") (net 34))
 (segment (start 110.6 49.4) (end 104.775 49.4) (width 0.2) (layer "F.Cu") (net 34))
 (segment (start 102.5 42.5) (end 100 40) (width 0.2) (layer "F.Cu") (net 34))
 (segment (start 112.42 47.58) (end 110.6 49.4) (width 0.2) (layer "F.Cu") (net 34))
 (via (at 100 40) (size 0.6) (drill 0.3) (layers "F.Cu" "B.Cu") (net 34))
 (via (at 102.5 52.5) (size 0.6) (drill 0.3) (layers "F.Cu" "B.Cu") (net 34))
 (segment (start 100 40) (end 99.4 40.6) (width 0.2) (layer "B.Cu") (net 34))
 (segment (start 99.4 40.6) (end 99.4 49.4) (width 0.2) (layer "B.Cu") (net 34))
 (segment (start 99.4 49.4) (end 102.5 52.5) (width 0.2) (layer "B.Cu") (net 34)))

